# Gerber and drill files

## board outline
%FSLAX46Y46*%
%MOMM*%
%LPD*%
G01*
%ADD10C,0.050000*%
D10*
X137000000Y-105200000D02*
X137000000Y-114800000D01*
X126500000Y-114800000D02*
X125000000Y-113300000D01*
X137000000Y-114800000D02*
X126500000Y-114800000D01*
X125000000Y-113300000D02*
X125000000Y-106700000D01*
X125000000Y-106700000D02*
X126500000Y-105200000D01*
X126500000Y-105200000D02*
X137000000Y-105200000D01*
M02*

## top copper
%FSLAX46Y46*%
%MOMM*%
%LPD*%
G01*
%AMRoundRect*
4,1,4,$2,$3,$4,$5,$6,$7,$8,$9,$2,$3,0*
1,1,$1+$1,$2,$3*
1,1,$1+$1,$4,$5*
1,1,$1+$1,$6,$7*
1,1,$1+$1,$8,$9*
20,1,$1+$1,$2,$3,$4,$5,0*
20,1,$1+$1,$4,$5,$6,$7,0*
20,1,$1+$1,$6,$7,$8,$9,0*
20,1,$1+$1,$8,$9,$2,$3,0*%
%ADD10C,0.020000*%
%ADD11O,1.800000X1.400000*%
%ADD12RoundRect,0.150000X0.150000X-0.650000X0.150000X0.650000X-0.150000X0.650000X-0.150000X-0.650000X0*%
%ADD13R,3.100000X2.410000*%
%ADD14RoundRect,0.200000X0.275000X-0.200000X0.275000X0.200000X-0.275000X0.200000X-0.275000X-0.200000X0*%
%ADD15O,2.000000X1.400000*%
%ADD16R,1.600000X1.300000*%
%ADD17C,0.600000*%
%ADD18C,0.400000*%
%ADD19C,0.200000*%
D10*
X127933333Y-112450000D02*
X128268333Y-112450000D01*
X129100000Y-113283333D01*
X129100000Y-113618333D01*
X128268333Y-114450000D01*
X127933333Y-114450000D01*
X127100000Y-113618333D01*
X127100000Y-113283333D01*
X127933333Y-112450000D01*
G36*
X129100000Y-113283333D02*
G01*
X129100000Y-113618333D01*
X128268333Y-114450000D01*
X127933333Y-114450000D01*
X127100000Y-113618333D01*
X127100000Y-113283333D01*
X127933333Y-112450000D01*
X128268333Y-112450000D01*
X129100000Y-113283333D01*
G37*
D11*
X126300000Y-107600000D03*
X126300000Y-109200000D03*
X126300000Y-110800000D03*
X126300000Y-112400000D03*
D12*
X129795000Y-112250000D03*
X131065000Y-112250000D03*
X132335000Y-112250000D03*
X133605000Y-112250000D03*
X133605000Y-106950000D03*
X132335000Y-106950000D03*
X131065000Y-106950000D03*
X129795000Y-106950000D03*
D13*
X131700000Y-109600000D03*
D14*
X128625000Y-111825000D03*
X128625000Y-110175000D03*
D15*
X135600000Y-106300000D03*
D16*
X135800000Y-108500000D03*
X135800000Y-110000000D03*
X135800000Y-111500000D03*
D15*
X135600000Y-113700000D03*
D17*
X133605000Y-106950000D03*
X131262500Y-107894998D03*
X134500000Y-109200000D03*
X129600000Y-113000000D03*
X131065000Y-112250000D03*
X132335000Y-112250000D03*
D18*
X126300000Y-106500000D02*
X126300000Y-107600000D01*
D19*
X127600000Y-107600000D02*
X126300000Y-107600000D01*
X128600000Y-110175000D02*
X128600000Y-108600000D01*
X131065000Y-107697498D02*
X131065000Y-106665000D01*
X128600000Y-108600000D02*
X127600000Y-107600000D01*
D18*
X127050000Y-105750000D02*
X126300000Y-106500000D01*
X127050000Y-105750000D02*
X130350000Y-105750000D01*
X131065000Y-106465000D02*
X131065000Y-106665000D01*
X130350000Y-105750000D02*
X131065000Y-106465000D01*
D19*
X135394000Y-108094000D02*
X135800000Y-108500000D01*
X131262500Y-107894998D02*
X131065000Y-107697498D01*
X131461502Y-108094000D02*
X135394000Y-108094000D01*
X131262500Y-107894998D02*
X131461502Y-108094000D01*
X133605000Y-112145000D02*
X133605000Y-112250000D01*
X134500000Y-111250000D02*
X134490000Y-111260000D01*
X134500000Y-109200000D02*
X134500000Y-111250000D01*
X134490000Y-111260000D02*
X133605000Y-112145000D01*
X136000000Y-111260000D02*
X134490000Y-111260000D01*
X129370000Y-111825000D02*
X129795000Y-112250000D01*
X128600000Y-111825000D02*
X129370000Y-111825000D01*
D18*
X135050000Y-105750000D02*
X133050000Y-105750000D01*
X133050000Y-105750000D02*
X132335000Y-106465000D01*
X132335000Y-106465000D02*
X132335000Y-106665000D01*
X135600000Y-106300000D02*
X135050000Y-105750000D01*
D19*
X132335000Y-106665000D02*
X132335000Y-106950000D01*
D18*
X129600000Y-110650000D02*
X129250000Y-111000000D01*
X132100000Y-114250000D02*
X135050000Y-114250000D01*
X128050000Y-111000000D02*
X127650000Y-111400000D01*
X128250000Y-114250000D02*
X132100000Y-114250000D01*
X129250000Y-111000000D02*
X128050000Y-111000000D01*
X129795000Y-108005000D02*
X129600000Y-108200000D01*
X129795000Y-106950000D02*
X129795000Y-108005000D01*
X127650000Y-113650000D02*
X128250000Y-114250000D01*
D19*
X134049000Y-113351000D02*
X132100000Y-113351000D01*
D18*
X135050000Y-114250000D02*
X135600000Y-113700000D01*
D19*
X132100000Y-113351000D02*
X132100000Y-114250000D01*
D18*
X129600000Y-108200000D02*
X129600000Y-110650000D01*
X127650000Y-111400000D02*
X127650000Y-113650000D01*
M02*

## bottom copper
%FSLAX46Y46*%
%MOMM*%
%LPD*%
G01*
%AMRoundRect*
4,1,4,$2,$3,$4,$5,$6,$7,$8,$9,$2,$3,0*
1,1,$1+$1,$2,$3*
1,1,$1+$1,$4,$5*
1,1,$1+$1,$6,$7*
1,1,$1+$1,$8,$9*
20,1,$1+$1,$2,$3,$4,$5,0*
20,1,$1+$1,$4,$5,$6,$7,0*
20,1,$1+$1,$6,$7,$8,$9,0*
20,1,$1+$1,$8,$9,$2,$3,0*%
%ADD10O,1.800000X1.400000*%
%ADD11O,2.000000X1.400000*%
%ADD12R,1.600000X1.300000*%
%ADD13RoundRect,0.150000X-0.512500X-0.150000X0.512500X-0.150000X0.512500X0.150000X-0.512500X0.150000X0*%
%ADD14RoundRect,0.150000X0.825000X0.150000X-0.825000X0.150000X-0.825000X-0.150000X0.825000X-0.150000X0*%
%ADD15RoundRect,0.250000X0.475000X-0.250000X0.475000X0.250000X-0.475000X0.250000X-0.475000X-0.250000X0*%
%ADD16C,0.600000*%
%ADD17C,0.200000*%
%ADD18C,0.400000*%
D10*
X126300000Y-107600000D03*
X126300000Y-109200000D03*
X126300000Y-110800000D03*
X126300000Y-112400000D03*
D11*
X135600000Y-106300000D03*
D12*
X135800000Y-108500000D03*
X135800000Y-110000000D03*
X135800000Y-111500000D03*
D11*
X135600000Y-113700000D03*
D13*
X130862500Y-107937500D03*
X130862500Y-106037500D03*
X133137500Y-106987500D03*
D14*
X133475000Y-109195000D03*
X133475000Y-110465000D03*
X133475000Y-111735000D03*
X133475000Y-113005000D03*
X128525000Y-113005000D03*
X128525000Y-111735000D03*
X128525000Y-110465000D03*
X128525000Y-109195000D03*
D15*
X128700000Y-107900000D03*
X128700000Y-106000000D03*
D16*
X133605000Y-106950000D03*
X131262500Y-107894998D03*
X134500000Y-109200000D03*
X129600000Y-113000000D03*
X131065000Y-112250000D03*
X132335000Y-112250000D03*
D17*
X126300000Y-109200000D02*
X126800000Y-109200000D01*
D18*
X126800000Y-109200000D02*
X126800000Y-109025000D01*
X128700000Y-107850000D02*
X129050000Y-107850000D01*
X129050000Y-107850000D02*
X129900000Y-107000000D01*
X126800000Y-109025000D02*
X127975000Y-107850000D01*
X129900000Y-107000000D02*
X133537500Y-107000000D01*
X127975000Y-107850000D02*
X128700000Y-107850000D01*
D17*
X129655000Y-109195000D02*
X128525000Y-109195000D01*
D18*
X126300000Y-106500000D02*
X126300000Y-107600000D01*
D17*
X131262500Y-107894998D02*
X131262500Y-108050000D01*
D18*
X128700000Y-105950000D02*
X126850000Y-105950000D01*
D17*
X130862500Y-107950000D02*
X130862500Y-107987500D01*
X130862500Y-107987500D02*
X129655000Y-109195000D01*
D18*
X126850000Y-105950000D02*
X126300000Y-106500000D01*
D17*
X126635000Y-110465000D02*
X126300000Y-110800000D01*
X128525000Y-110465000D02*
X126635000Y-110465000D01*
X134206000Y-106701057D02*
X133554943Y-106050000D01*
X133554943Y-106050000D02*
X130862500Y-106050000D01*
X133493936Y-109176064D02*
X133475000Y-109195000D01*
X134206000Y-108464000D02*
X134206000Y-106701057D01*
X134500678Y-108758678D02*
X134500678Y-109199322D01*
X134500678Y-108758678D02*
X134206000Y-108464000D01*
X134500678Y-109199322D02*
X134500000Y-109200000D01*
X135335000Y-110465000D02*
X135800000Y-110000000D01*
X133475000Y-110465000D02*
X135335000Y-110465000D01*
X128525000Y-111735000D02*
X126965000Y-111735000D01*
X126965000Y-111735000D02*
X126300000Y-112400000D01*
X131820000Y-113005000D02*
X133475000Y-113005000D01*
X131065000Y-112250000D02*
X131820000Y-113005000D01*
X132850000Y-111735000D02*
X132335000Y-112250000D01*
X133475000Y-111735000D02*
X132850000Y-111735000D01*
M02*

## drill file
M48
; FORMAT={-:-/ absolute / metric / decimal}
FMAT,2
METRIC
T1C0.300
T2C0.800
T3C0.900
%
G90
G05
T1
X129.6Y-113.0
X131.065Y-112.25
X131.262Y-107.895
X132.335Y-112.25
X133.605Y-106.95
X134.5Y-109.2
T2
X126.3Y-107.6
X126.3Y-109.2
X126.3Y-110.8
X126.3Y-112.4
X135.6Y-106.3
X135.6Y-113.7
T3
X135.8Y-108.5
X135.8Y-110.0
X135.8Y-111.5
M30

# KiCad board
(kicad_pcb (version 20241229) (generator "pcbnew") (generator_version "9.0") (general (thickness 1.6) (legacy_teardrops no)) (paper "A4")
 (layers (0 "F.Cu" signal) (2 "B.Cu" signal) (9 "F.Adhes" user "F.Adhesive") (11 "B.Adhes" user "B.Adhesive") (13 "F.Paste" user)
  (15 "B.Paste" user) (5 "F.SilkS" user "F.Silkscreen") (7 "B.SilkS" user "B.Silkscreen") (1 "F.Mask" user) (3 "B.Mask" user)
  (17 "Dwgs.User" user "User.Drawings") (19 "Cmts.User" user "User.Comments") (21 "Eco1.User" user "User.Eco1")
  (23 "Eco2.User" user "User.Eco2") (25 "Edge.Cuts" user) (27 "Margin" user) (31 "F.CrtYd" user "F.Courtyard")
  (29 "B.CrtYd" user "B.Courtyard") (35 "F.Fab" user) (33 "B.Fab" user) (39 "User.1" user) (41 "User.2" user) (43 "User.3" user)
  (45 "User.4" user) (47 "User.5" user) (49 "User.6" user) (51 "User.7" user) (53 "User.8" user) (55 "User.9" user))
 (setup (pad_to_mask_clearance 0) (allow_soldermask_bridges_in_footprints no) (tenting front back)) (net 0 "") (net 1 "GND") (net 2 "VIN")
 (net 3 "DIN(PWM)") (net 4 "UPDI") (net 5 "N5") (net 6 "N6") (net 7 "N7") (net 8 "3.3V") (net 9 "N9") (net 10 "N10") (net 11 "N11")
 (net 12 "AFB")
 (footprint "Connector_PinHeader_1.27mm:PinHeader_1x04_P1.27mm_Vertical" (layer "F.Cu") (at 126 110)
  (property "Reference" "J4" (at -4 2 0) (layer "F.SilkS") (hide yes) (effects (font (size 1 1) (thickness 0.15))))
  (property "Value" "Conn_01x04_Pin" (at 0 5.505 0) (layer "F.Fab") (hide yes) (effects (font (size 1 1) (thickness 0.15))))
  (pad "1" thru_hole oval (at 0.3 -2.4) (size 1.8 1.4) (drill 0.8) (layers "*.Cu" "*.Mask") (remove_unused_layers no) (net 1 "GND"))
  (pad "2" thru_hole oval (at 0.3 -0.8) (size 1.8 1.4) (drill 0.8) (layers "*.Cu" "*.Mask") (remove_unused_layers no) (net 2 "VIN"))
  (pad "3" thru_hole oval (at 0.3 0.8) (size 1.8 1.4) (drill 0.8) (layers "*.Cu" "*.Mask") (remove_unused_layers no) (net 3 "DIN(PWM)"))
  (pad "4" thru_hole oval (at 0.3 2.4) (size 1.8 1.4) (drill 0.8) (layers "*.Cu" "*.Mask") (remove_unused_layers no) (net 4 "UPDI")))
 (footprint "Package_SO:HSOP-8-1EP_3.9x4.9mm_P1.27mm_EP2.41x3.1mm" (layer "F.Cu") (at 131.7 109.6 90)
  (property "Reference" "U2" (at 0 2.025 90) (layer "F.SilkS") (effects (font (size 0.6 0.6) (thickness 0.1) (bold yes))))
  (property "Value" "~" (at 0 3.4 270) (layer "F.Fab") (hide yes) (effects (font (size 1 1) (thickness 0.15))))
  (pad "" smd roundrect (at -0.6 -0.775 90) (size 0.97 1.25) (layers "F.Paste") (roundrect_rratio 0.25))
  (pad "" smd roundrect (at -0.6 0.775 90) (size 0.97 1.25) (layers "F.Paste") (roundrect_rratio 0.25))
  (pad "" smd roundrect (at 0.6 -0.775 90) (size 0.97 1.25) (layers "F.Paste") (roundrect_rratio 0.25))
  (pad "" smd roundrect (at 0.6 0.775 90) (size 0.97 1.25) (layers "F.Paste") (roundrect_rratio 0.25))
  (pad "1" smd roundrect (at -2.65 -1.905 90) (size 1.6 0.6) (layers "F.Cu" "F.Mask" "F.Paste") (roundrect_rratio 0.25) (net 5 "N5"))
  (pad "2" smd roundrect (at -2.65 -0.635 90) (size 1.6 0.6) (layers "F.Cu" "F.Mask" "F.Paste") (roundrect_rratio 0.25) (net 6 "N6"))
  (pad "3" smd roundrect (at -2.65 0.635 90) (size 1.6 0.6) (layers "F.Cu" "F.Mask" "F.Paste") (roundrect_rratio 0.25) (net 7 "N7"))
  (pad "4" smd roundrect (at -2.65 1.905 90) (size 1.6 0.6) (layers "F.Cu" "F.Mask" "F.Paste") (roundrect_rratio 0.25) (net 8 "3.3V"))
  (pad "5" smd roundrect (at 2.65 1.905 90) (size 1.6 0.6) (layers "F.Cu" "F.Mask" "F.Paste") (roundrect_rratio 0.25) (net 2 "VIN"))
  (pad "6" smd roundrect (at 2.65 0.635 90) (size 1.6 0.6) (layers "F.Cu" "F.Mask" "F.Paste") (roundrect_rratio 0.25) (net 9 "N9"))
  (pad "7" smd roundrect (at 2.65 -0.635 90) (size 1.6 0.6) (layers "F.Cu" "F.Mask" "F.Paste") (roundrect_rratio 0.25) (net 1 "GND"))
  (pad "8" smd roundrect (at 2.65 -1.905 90) (size 1.6 0.6) (layers "F.Cu" "F.Mask" "F.Paste") (roundrect_rratio 0.25) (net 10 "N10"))
  (pad "9" smd rect (at 0 0 90) (size 2.41 3.1) (layers "F.Cu" "F.Mask") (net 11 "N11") (zone_connect 2)))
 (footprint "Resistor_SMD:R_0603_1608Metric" (layer "F.Cu") (at 128.625 111 90)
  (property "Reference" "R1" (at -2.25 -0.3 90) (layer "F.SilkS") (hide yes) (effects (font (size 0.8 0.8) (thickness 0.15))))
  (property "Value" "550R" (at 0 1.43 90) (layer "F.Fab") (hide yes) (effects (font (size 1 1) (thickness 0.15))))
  (pad "1" smd roundrect (at -0.825 0 90) (size 0.8 0.95) (layers "F.Cu" "F.Mask" "F.Paste") (roundrect_rratio 0.25) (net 5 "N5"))
  (pad "2" smd roundrect (at 0.825 0 90) (size 0.8 0.95) (layers "F.Cu" "F.Mask" "F.Paste") (roundrect_rratio 0.25) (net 1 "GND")))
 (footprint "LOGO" (layer "F.Cu") (at 128.1 113.45)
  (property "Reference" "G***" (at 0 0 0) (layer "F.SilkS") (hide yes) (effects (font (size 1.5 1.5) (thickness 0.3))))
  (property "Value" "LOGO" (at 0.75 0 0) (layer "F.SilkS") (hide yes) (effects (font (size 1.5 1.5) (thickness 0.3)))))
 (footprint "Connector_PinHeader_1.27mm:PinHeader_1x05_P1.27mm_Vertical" (layer "F.Cu") (at 136 110)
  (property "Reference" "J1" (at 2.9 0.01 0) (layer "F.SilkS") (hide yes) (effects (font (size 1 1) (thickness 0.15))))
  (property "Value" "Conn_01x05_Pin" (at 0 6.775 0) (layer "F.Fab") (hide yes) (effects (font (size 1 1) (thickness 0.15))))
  (pad "1" thru_hole oval (at -0.4 -3.7) (size 2 1.4) (drill 0.8) (layers "*.Cu" "*.Mask") (remove_unused_layers no) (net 9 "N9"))
  (pad "2" thru_hole rect (at -0.2 -1.5) (size 1.6 1.3) (drill 0.9) (layers "*.Cu" "*.Mask") (remove_unused_layers no) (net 1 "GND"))
  (pad "3" thru_hole rect (at -0.2 0) (size 1.6 1.3) (drill 0.9) (layers "*.Cu" "*.Mask") (remove_unused_layers no) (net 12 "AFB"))
  (pad "4" thru_hole rect (at -0.2 1.5) (size 1.6 1.3) (drill 0.9) (layers "*.Cu" "*.Mask") (remove_unused_layers no) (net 8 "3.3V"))
  (pad "5" thru_hole oval (at -0.4 3.7) (size 2 1.4) (drill 0.8) (layers "*.Cu" "*.Mask") (remove_unused_layers no) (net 10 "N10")))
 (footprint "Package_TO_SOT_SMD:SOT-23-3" (layer "B.Cu") (at 132 106.9875)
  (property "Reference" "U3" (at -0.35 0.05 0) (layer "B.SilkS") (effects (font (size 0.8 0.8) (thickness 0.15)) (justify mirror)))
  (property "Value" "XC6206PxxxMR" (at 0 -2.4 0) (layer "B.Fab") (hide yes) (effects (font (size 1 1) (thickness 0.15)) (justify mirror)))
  (pad "1" smd roundrect (at -1.1375 0.95) (size 1.325 0.6) (layers "B.Cu" "B.Mask" "B.Paste") (roundrect_rratio 0.25) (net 1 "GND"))
  (pad "2" smd roundrect (at -1.1375 -0.95) (size 1.325 0.6) (layers "B.Cu" "B.Mask" "B.Paste") (roundrect_rratio 0.25) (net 8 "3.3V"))
  (pad "3" smd roundrect (at 1.1375 0) (size 1.325 0.6) (layers "B.Cu" "B.Mask" "B.Paste") (roundrect_rratio 0.25) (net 2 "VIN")))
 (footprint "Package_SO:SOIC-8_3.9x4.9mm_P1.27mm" (layer "B.Cu") (at 131 111.1 180)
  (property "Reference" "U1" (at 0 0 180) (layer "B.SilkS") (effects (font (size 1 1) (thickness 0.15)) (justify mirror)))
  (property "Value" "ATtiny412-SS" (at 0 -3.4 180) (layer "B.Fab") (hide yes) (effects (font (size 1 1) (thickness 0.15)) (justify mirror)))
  (pad "1" smd roundrect (at -2.475 1.905 180) (size 1.95 0.6) (layers "B.Cu" "B.Mask" "B.Paste") (roundrect_rratio 0.25) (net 8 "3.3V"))
  (pad "2" smd roundrect (at -2.475 0.635 180) (size 1.95 0.6) (layers "B.Cu" "B.Mask" "B.Paste") (roundrect_rratio 0.25) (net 12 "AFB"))
  (pad "3" smd roundrect (at -2.475 -0.635 180) (size 1.95 0.6) (layers "B.Cu" "B.Mask" "B.Paste") (roundrect_rratio 0.25) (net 7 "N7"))
  (pad "4" smd roundrect (at -2.475 -1.905 180) (size 1.95 0.6) (layers "B.Cu" "B.Mask" "B.Paste") (roundrect_rratio 0.25) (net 6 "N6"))
  (pad "5" smd roundrect (at 2.475 -1.905 180) (size 1.95 0.6) (layers "B.Cu" "B.Mask" "B.Paste") (roundrect_rratio 0.25) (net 5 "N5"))
  (pad "6" smd roundrect (at 2.475 -0.635 180) (size 1.95 0.6) (layers "B.Cu" "B.Mask" "B.Paste") (roundrect_rratio 0.25) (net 4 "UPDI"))
  (pad "7" smd roundrect (at 2.475 0.635 180) (size 1.95 0.6) (layers "B.Cu" "B.Mask" "B.Paste") (roundrect_rratio 0.25) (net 3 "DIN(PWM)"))
  (pad "8" smd roundrect (at 2.475 1.905 180) (size 1.95 0.6) (layers "B.Cu" "B.Mask" "B.Paste") (roundrect_rratio 0.25) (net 1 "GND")))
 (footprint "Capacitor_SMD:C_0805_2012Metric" (layer "B.Cu") (at 128.7 106.95 90)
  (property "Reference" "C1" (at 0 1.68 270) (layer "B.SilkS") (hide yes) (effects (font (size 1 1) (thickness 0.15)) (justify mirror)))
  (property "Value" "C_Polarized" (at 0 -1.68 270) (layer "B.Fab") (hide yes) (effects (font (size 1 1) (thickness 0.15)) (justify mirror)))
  (pad "1" smd roundrect (at -0.95 0 90) (size 1 1.45) (layers "B.Cu" "B.Mask" "B.Paste") (roundrect_rratio 0.25) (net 2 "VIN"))
  (pad "2" smd roundrect (at 0.95 0 90) (size 1 1.45) (layers "B.Cu" "B.Mask" "B.Paste") (roundrect_rratio 0.25) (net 1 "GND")))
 (gr_poly
  (pts (xy 127.933333 112.45) (xy 128.268333 112.45) (xy 129.1 113.283333) (xy 129.1 113.618333) (xy 128.268333 114.45)
   (xy 127.933333 114.45) (xy 127.1 113.618333) (xy 127.1 113.283333))
  (stroke (width 0.02) (type solid)) (fill yes) (layer "F.Cu") (net 10))
 (gr_line (start 137 105.2) (end 137 114.8) (stroke (width 0.05) (type default)) (layer "Edge.Cuts"))
 (gr_line (start 126.5 114.8) (end 125 113.3) (stroke (width 0.05) (type default)) (layer "Edge.Cuts"))
 (gr_line (start 137 114.8) (end 126.5 114.8) (stroke (width 0.05) (type default)) (layer "Edge.Cuts"))
 (gr_line (start 125 113.3) (end 125 106.7) (stroke (width 0.05) (type default)) (layer "Edge.Cuts"))
 (gr_line (start 125 106.7) (end 126.5 105.2) (stroke (width 0.05) (type default)) (layer "Edge.Cuts"))
 (gr_line (start 126.5 105.2) (end 137 105.2) (stroke (width 0.05) (type default)) (layer "Edge.Cuts"))
 (via (at 133.605 106.95) (size 0.6) (drill 0.3) (layers "F.Cu" "B.Cu") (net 2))
 (segment (start 126.3 109.2) (end 126.8 109.2) (width 0.2) (layer "B.Cu") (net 2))
 (segment (start 126.8 109.2) (end 126.8 109.025) (width 0.4) (layer "B.Cu") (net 2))
 (segment (start 128.7 107.85) (end 129.05 107.85) (width 0.4) (layer "B.Cu") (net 2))
 (segment (start 129.05 107.85) (end 129.9 107) (width 0.4) (layer "B.Cu") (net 2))
 (segment (start 126.8 109.025) (end 127.975 107.85) (width 0.4) (layer "B.Cu") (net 2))
 (segment (start 129.9 107) (end 133.5375 107) (width 0.4) (layer "B.Cu") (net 2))
 (segment (start 127.975 107.85) (end 128.7 107.85) (width 0.4) (layer "B.Cu") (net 2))
 (segment (start 126.3 106.5) (end 126.3 107.6) (width 0.4) (layer "F.Cu") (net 1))
 (segment (start 127.6 107.6) (end 126.3 107.6) (width 0.2) (layer "F.Cu") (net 1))
 (segment (start 128.6 110.175) (end 128.6 108.6) (width 0.2) (layer "F.Cu") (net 1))
 (segment (start 131.065 107.697498) (end 131.065 106.665) (width 0.2) (layer "F.Cu") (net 1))
 (segment (start 128.6 108.6) (end 127.6 107.6) (width 0.2) (layer "F.Cu") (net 1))
 (segment (start 127.05 105.75) (end 126.3 106.5) (width 0.4) (layer "F.Cu") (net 1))
 (segment (start 127.05 105.75) (end 130.35 105.75) (width 0.4) (layer "F.Cu") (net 1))
 (segment (start 131.065 106.465) (end 131.065 106.665) (width 0.4) (layer "F.Cu") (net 1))
 (segment (start 130.35 105.75) (end 131.065 106.465) (width 0.4) (layer "F.Cu") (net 1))
 (segment (start 135.394 108.094) (end 135.8 108.5) (width 0.2) (layer "F.Cu") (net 1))
 (segment (start 131.2625 107.894998) (end 131.065 107.697498) (width 0.2) (layer "F.Cu") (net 1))
 (segment (start 131.461502 108.094) (end 135.394 108.094) (width 0.2) (layer "F.Cu") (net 1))
 (segment (start 131.2625 107.894998) (end 131.461502 108.094) (width 0.2) (layer "F.Cu") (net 1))
 (via (at 131.2625 107.894998) (size 0.6) (drill 0.3) (layers "F.Cu" "B.Cu") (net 1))
 (segment (start 129.655 109.195) (end 128.525 109.195) (width 0.2) (layer "B.Cu") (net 1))
 (segment (start 126.3 106.5) (end 126.3 107.6) (width 0.4) (layer "B.Cu") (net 1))
 (segment (start 131.2625 107.894998) (end 131.2625 108.05) (width 0.2) (layer "B.Cu") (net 1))
 (segment (start 128.7 105.95) (end 126.85 105.95) (width 0.4) (layer "B.Cu") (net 1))
 (segment (start 130.8625 107.95) (end 130.8625 107.9875) (width 0.2) (layer "B.Cu") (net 1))
 (segment (start 130.8625 107.9875) (end 129.655 109.195) (width 0.2) (layer "B.Cu") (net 1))
 (segment (start 126.85 105.95) (end 126.3 106.5) (width 0.4) (layer "B.Cu") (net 1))
 (segment (start 126.635 110.465) (end 126.3 110.8) (width 0.2) (layer "B.Cu") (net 3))
 (segment (start 128.525 110.465) (end 126.635 110.465) (width 0.2) (layer "B.Cu") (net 3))
 (segment (start 133.605 112.145) (end 133.605 112.25) (width 0.2) (layer "F.Cu") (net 8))
 (segment (start 134.5 111.25) (end 134.49 111.26) (width 0.2) (layer "F.Cu") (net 8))
 (segment (start 134.5 109.2) (end 134.5 111.25) (width 0.2) (layer "F.Cu") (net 8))
 (segment (start 134.49 111.26) (end 133.605 112.145) (width 0.2) (layer "F.Cu") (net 8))
 (segment (start 136 111.26) (end 134.49 111.26) (width 0.2) (layer "F.Cu") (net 8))
 (via (at 134.5 109.2) (size 0.6) (drill 0.3) (layers "F.Cu" "B.Cu") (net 8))
 (segment (start 134.206 106.701057) (end 133.554943 106.05) (width 0.2) (layer "B.Cu") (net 8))
 (segment (start 133.554943 106.05) (end 130.8625 106.05) (width 0.2) (layer "B.Cu") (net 8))
 (segment (start 133.493936 109.176064) (end 133.475 109.195) (width 0.2) (layer "B.Cu") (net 8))
 (segment (start 134.206 108.464) (end 134.206 106.701057) (width 0.2) (layer "B.Cu") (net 8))
 (segment (start 134.500678 108.758678) (end 134.500678 109.199322) (width 0.2) (layer "B.Cu") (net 8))
 (segment (start 134.500678 108.758678) (end 134.206 108.464) (width 0.2) (layer "B.Cu") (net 8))
 (segment (start 134.500678 109.199322) (end 134.5 109.2) (width 0.2) (layer "B.Cu") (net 8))
 (segment (start 135.335 110.465) (end 135.8 110) (width 0.2) (layer "B.Cu") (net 12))
 (segment (start 133.475 110.465) (end 135.335 110.465) (width 0.2) (layer "B.Cu") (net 12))
 (segment (start 128.525 111.735) (end 126.965 111.735) (width 0.2) (layer "B.Cu") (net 4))
 (segment (start 126.965 111.735) (end 126.3 112.4) (width 0.2) (layer "B.Cu") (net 4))
 (segment (start 129.37 111.825) (end 129.795 112.25) (width 0.2) (layer "F.Cu") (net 5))
 (segment (start 128.6 111.825) (end 129.37 111.825) (width 0.2) (layer "F.Cu") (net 5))
 (via (at 129.6 113) (size 0.6) (drill 0.3) (layers "F.Cu" "B.Cu") (free yes) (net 5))
 (via (at 131.065 112.25) (size 0.6) (drill 0.3) (layers "F.Cu" "B.Cu") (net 6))
 (segment (start 131.82 113.005) (end 133.475 113.005) (width 0.2) (layer "B.Cu") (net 6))
 (segment (start 131.065 112.25) (end 131.82 113.005) (width 0.2) (layer "B.Cu") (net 6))
 (via (at 132.335 112.25) (size 0.6) (drill 0.3) (layers "F.Cu" "B.Cu") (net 7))
 (segment (start 132.85 111.735) (end 132.335 112.25) (width 0.2) (layer "B.Cu") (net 7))
 (segment (start 133.475 111.735) (end 132.85 111.735) (width 0.2) (layer "B.Cu") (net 7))
 (segment (start 135.05 105.75) (end 133.05 105.75) (width 0.4) (layer "F.Cu") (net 9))
 (segment (start 133.05 105.75) (end 132.335 106.465) (width 0.4) (layer "F.Cu") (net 9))
 (segment (start 132.335 106.465) (end 132.335 106.665) (width 0.4) (layer "F.Cu") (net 9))
 (segment (start 135.6 106.3) (end 135.05 105.75) (width 0.4) (layer "F.Cu") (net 9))
 (segment (start 132.335 106.665) (end 132.335 106.95) (width 0.2) (layer "F.Cu") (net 9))
 (segment (start 129.6 110.65) (end 129.25 111) (width 0.4) (layer "F.Cu") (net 10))
 (segment (start 132.1 114.25) (end 135.05 114.25) (width 0.4) (layer "F.Cu") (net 10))
 (segment (start 128.05 111) (end 127.65 111.4) (width 0.4) (layer "F.Cu") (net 10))
 (segment (start 128.25 114.25) (end 132.1 114.25) (width 0.4) (layer "F.Cu") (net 10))
 (segment (start 129.25 111) (end 128.05 111) (width 0.4) (layer "F.Cu") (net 10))
 (segment (start 129.795 108.005) (end 129.6 108.2) (width 0.4) (layer "F.Cu") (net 10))
 (segment (start 129.795 106.95) (end 129.795 108.005) (width 0.4) (layer "F.Cu") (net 10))
 (segment (start 127.65 113.65) (end 128.25 114.25) (width 0.4) (layer "F.Cu") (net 10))
 (segment (start 134.049 113.351) (end 132.1 113.351) (width 0.2) (layer "F.Cu") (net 10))
 (segment (start 135.05 114.25) (end 135.6 113.7) (width 0.4) (layer "F.Cu") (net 10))
 (segment (start 132.1 113.351) (end 132.1 114.25) (width 0.2) (layer "F.Cu") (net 10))
 (segment (start 129.6 108.2) (end 129.6 110.65) (width 0.4) (layer "F.Cu") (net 10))
 (segment (start 127.65 111.4) (end 127.65 113.65) (width 0.4) (layer "F.Cu") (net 10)))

